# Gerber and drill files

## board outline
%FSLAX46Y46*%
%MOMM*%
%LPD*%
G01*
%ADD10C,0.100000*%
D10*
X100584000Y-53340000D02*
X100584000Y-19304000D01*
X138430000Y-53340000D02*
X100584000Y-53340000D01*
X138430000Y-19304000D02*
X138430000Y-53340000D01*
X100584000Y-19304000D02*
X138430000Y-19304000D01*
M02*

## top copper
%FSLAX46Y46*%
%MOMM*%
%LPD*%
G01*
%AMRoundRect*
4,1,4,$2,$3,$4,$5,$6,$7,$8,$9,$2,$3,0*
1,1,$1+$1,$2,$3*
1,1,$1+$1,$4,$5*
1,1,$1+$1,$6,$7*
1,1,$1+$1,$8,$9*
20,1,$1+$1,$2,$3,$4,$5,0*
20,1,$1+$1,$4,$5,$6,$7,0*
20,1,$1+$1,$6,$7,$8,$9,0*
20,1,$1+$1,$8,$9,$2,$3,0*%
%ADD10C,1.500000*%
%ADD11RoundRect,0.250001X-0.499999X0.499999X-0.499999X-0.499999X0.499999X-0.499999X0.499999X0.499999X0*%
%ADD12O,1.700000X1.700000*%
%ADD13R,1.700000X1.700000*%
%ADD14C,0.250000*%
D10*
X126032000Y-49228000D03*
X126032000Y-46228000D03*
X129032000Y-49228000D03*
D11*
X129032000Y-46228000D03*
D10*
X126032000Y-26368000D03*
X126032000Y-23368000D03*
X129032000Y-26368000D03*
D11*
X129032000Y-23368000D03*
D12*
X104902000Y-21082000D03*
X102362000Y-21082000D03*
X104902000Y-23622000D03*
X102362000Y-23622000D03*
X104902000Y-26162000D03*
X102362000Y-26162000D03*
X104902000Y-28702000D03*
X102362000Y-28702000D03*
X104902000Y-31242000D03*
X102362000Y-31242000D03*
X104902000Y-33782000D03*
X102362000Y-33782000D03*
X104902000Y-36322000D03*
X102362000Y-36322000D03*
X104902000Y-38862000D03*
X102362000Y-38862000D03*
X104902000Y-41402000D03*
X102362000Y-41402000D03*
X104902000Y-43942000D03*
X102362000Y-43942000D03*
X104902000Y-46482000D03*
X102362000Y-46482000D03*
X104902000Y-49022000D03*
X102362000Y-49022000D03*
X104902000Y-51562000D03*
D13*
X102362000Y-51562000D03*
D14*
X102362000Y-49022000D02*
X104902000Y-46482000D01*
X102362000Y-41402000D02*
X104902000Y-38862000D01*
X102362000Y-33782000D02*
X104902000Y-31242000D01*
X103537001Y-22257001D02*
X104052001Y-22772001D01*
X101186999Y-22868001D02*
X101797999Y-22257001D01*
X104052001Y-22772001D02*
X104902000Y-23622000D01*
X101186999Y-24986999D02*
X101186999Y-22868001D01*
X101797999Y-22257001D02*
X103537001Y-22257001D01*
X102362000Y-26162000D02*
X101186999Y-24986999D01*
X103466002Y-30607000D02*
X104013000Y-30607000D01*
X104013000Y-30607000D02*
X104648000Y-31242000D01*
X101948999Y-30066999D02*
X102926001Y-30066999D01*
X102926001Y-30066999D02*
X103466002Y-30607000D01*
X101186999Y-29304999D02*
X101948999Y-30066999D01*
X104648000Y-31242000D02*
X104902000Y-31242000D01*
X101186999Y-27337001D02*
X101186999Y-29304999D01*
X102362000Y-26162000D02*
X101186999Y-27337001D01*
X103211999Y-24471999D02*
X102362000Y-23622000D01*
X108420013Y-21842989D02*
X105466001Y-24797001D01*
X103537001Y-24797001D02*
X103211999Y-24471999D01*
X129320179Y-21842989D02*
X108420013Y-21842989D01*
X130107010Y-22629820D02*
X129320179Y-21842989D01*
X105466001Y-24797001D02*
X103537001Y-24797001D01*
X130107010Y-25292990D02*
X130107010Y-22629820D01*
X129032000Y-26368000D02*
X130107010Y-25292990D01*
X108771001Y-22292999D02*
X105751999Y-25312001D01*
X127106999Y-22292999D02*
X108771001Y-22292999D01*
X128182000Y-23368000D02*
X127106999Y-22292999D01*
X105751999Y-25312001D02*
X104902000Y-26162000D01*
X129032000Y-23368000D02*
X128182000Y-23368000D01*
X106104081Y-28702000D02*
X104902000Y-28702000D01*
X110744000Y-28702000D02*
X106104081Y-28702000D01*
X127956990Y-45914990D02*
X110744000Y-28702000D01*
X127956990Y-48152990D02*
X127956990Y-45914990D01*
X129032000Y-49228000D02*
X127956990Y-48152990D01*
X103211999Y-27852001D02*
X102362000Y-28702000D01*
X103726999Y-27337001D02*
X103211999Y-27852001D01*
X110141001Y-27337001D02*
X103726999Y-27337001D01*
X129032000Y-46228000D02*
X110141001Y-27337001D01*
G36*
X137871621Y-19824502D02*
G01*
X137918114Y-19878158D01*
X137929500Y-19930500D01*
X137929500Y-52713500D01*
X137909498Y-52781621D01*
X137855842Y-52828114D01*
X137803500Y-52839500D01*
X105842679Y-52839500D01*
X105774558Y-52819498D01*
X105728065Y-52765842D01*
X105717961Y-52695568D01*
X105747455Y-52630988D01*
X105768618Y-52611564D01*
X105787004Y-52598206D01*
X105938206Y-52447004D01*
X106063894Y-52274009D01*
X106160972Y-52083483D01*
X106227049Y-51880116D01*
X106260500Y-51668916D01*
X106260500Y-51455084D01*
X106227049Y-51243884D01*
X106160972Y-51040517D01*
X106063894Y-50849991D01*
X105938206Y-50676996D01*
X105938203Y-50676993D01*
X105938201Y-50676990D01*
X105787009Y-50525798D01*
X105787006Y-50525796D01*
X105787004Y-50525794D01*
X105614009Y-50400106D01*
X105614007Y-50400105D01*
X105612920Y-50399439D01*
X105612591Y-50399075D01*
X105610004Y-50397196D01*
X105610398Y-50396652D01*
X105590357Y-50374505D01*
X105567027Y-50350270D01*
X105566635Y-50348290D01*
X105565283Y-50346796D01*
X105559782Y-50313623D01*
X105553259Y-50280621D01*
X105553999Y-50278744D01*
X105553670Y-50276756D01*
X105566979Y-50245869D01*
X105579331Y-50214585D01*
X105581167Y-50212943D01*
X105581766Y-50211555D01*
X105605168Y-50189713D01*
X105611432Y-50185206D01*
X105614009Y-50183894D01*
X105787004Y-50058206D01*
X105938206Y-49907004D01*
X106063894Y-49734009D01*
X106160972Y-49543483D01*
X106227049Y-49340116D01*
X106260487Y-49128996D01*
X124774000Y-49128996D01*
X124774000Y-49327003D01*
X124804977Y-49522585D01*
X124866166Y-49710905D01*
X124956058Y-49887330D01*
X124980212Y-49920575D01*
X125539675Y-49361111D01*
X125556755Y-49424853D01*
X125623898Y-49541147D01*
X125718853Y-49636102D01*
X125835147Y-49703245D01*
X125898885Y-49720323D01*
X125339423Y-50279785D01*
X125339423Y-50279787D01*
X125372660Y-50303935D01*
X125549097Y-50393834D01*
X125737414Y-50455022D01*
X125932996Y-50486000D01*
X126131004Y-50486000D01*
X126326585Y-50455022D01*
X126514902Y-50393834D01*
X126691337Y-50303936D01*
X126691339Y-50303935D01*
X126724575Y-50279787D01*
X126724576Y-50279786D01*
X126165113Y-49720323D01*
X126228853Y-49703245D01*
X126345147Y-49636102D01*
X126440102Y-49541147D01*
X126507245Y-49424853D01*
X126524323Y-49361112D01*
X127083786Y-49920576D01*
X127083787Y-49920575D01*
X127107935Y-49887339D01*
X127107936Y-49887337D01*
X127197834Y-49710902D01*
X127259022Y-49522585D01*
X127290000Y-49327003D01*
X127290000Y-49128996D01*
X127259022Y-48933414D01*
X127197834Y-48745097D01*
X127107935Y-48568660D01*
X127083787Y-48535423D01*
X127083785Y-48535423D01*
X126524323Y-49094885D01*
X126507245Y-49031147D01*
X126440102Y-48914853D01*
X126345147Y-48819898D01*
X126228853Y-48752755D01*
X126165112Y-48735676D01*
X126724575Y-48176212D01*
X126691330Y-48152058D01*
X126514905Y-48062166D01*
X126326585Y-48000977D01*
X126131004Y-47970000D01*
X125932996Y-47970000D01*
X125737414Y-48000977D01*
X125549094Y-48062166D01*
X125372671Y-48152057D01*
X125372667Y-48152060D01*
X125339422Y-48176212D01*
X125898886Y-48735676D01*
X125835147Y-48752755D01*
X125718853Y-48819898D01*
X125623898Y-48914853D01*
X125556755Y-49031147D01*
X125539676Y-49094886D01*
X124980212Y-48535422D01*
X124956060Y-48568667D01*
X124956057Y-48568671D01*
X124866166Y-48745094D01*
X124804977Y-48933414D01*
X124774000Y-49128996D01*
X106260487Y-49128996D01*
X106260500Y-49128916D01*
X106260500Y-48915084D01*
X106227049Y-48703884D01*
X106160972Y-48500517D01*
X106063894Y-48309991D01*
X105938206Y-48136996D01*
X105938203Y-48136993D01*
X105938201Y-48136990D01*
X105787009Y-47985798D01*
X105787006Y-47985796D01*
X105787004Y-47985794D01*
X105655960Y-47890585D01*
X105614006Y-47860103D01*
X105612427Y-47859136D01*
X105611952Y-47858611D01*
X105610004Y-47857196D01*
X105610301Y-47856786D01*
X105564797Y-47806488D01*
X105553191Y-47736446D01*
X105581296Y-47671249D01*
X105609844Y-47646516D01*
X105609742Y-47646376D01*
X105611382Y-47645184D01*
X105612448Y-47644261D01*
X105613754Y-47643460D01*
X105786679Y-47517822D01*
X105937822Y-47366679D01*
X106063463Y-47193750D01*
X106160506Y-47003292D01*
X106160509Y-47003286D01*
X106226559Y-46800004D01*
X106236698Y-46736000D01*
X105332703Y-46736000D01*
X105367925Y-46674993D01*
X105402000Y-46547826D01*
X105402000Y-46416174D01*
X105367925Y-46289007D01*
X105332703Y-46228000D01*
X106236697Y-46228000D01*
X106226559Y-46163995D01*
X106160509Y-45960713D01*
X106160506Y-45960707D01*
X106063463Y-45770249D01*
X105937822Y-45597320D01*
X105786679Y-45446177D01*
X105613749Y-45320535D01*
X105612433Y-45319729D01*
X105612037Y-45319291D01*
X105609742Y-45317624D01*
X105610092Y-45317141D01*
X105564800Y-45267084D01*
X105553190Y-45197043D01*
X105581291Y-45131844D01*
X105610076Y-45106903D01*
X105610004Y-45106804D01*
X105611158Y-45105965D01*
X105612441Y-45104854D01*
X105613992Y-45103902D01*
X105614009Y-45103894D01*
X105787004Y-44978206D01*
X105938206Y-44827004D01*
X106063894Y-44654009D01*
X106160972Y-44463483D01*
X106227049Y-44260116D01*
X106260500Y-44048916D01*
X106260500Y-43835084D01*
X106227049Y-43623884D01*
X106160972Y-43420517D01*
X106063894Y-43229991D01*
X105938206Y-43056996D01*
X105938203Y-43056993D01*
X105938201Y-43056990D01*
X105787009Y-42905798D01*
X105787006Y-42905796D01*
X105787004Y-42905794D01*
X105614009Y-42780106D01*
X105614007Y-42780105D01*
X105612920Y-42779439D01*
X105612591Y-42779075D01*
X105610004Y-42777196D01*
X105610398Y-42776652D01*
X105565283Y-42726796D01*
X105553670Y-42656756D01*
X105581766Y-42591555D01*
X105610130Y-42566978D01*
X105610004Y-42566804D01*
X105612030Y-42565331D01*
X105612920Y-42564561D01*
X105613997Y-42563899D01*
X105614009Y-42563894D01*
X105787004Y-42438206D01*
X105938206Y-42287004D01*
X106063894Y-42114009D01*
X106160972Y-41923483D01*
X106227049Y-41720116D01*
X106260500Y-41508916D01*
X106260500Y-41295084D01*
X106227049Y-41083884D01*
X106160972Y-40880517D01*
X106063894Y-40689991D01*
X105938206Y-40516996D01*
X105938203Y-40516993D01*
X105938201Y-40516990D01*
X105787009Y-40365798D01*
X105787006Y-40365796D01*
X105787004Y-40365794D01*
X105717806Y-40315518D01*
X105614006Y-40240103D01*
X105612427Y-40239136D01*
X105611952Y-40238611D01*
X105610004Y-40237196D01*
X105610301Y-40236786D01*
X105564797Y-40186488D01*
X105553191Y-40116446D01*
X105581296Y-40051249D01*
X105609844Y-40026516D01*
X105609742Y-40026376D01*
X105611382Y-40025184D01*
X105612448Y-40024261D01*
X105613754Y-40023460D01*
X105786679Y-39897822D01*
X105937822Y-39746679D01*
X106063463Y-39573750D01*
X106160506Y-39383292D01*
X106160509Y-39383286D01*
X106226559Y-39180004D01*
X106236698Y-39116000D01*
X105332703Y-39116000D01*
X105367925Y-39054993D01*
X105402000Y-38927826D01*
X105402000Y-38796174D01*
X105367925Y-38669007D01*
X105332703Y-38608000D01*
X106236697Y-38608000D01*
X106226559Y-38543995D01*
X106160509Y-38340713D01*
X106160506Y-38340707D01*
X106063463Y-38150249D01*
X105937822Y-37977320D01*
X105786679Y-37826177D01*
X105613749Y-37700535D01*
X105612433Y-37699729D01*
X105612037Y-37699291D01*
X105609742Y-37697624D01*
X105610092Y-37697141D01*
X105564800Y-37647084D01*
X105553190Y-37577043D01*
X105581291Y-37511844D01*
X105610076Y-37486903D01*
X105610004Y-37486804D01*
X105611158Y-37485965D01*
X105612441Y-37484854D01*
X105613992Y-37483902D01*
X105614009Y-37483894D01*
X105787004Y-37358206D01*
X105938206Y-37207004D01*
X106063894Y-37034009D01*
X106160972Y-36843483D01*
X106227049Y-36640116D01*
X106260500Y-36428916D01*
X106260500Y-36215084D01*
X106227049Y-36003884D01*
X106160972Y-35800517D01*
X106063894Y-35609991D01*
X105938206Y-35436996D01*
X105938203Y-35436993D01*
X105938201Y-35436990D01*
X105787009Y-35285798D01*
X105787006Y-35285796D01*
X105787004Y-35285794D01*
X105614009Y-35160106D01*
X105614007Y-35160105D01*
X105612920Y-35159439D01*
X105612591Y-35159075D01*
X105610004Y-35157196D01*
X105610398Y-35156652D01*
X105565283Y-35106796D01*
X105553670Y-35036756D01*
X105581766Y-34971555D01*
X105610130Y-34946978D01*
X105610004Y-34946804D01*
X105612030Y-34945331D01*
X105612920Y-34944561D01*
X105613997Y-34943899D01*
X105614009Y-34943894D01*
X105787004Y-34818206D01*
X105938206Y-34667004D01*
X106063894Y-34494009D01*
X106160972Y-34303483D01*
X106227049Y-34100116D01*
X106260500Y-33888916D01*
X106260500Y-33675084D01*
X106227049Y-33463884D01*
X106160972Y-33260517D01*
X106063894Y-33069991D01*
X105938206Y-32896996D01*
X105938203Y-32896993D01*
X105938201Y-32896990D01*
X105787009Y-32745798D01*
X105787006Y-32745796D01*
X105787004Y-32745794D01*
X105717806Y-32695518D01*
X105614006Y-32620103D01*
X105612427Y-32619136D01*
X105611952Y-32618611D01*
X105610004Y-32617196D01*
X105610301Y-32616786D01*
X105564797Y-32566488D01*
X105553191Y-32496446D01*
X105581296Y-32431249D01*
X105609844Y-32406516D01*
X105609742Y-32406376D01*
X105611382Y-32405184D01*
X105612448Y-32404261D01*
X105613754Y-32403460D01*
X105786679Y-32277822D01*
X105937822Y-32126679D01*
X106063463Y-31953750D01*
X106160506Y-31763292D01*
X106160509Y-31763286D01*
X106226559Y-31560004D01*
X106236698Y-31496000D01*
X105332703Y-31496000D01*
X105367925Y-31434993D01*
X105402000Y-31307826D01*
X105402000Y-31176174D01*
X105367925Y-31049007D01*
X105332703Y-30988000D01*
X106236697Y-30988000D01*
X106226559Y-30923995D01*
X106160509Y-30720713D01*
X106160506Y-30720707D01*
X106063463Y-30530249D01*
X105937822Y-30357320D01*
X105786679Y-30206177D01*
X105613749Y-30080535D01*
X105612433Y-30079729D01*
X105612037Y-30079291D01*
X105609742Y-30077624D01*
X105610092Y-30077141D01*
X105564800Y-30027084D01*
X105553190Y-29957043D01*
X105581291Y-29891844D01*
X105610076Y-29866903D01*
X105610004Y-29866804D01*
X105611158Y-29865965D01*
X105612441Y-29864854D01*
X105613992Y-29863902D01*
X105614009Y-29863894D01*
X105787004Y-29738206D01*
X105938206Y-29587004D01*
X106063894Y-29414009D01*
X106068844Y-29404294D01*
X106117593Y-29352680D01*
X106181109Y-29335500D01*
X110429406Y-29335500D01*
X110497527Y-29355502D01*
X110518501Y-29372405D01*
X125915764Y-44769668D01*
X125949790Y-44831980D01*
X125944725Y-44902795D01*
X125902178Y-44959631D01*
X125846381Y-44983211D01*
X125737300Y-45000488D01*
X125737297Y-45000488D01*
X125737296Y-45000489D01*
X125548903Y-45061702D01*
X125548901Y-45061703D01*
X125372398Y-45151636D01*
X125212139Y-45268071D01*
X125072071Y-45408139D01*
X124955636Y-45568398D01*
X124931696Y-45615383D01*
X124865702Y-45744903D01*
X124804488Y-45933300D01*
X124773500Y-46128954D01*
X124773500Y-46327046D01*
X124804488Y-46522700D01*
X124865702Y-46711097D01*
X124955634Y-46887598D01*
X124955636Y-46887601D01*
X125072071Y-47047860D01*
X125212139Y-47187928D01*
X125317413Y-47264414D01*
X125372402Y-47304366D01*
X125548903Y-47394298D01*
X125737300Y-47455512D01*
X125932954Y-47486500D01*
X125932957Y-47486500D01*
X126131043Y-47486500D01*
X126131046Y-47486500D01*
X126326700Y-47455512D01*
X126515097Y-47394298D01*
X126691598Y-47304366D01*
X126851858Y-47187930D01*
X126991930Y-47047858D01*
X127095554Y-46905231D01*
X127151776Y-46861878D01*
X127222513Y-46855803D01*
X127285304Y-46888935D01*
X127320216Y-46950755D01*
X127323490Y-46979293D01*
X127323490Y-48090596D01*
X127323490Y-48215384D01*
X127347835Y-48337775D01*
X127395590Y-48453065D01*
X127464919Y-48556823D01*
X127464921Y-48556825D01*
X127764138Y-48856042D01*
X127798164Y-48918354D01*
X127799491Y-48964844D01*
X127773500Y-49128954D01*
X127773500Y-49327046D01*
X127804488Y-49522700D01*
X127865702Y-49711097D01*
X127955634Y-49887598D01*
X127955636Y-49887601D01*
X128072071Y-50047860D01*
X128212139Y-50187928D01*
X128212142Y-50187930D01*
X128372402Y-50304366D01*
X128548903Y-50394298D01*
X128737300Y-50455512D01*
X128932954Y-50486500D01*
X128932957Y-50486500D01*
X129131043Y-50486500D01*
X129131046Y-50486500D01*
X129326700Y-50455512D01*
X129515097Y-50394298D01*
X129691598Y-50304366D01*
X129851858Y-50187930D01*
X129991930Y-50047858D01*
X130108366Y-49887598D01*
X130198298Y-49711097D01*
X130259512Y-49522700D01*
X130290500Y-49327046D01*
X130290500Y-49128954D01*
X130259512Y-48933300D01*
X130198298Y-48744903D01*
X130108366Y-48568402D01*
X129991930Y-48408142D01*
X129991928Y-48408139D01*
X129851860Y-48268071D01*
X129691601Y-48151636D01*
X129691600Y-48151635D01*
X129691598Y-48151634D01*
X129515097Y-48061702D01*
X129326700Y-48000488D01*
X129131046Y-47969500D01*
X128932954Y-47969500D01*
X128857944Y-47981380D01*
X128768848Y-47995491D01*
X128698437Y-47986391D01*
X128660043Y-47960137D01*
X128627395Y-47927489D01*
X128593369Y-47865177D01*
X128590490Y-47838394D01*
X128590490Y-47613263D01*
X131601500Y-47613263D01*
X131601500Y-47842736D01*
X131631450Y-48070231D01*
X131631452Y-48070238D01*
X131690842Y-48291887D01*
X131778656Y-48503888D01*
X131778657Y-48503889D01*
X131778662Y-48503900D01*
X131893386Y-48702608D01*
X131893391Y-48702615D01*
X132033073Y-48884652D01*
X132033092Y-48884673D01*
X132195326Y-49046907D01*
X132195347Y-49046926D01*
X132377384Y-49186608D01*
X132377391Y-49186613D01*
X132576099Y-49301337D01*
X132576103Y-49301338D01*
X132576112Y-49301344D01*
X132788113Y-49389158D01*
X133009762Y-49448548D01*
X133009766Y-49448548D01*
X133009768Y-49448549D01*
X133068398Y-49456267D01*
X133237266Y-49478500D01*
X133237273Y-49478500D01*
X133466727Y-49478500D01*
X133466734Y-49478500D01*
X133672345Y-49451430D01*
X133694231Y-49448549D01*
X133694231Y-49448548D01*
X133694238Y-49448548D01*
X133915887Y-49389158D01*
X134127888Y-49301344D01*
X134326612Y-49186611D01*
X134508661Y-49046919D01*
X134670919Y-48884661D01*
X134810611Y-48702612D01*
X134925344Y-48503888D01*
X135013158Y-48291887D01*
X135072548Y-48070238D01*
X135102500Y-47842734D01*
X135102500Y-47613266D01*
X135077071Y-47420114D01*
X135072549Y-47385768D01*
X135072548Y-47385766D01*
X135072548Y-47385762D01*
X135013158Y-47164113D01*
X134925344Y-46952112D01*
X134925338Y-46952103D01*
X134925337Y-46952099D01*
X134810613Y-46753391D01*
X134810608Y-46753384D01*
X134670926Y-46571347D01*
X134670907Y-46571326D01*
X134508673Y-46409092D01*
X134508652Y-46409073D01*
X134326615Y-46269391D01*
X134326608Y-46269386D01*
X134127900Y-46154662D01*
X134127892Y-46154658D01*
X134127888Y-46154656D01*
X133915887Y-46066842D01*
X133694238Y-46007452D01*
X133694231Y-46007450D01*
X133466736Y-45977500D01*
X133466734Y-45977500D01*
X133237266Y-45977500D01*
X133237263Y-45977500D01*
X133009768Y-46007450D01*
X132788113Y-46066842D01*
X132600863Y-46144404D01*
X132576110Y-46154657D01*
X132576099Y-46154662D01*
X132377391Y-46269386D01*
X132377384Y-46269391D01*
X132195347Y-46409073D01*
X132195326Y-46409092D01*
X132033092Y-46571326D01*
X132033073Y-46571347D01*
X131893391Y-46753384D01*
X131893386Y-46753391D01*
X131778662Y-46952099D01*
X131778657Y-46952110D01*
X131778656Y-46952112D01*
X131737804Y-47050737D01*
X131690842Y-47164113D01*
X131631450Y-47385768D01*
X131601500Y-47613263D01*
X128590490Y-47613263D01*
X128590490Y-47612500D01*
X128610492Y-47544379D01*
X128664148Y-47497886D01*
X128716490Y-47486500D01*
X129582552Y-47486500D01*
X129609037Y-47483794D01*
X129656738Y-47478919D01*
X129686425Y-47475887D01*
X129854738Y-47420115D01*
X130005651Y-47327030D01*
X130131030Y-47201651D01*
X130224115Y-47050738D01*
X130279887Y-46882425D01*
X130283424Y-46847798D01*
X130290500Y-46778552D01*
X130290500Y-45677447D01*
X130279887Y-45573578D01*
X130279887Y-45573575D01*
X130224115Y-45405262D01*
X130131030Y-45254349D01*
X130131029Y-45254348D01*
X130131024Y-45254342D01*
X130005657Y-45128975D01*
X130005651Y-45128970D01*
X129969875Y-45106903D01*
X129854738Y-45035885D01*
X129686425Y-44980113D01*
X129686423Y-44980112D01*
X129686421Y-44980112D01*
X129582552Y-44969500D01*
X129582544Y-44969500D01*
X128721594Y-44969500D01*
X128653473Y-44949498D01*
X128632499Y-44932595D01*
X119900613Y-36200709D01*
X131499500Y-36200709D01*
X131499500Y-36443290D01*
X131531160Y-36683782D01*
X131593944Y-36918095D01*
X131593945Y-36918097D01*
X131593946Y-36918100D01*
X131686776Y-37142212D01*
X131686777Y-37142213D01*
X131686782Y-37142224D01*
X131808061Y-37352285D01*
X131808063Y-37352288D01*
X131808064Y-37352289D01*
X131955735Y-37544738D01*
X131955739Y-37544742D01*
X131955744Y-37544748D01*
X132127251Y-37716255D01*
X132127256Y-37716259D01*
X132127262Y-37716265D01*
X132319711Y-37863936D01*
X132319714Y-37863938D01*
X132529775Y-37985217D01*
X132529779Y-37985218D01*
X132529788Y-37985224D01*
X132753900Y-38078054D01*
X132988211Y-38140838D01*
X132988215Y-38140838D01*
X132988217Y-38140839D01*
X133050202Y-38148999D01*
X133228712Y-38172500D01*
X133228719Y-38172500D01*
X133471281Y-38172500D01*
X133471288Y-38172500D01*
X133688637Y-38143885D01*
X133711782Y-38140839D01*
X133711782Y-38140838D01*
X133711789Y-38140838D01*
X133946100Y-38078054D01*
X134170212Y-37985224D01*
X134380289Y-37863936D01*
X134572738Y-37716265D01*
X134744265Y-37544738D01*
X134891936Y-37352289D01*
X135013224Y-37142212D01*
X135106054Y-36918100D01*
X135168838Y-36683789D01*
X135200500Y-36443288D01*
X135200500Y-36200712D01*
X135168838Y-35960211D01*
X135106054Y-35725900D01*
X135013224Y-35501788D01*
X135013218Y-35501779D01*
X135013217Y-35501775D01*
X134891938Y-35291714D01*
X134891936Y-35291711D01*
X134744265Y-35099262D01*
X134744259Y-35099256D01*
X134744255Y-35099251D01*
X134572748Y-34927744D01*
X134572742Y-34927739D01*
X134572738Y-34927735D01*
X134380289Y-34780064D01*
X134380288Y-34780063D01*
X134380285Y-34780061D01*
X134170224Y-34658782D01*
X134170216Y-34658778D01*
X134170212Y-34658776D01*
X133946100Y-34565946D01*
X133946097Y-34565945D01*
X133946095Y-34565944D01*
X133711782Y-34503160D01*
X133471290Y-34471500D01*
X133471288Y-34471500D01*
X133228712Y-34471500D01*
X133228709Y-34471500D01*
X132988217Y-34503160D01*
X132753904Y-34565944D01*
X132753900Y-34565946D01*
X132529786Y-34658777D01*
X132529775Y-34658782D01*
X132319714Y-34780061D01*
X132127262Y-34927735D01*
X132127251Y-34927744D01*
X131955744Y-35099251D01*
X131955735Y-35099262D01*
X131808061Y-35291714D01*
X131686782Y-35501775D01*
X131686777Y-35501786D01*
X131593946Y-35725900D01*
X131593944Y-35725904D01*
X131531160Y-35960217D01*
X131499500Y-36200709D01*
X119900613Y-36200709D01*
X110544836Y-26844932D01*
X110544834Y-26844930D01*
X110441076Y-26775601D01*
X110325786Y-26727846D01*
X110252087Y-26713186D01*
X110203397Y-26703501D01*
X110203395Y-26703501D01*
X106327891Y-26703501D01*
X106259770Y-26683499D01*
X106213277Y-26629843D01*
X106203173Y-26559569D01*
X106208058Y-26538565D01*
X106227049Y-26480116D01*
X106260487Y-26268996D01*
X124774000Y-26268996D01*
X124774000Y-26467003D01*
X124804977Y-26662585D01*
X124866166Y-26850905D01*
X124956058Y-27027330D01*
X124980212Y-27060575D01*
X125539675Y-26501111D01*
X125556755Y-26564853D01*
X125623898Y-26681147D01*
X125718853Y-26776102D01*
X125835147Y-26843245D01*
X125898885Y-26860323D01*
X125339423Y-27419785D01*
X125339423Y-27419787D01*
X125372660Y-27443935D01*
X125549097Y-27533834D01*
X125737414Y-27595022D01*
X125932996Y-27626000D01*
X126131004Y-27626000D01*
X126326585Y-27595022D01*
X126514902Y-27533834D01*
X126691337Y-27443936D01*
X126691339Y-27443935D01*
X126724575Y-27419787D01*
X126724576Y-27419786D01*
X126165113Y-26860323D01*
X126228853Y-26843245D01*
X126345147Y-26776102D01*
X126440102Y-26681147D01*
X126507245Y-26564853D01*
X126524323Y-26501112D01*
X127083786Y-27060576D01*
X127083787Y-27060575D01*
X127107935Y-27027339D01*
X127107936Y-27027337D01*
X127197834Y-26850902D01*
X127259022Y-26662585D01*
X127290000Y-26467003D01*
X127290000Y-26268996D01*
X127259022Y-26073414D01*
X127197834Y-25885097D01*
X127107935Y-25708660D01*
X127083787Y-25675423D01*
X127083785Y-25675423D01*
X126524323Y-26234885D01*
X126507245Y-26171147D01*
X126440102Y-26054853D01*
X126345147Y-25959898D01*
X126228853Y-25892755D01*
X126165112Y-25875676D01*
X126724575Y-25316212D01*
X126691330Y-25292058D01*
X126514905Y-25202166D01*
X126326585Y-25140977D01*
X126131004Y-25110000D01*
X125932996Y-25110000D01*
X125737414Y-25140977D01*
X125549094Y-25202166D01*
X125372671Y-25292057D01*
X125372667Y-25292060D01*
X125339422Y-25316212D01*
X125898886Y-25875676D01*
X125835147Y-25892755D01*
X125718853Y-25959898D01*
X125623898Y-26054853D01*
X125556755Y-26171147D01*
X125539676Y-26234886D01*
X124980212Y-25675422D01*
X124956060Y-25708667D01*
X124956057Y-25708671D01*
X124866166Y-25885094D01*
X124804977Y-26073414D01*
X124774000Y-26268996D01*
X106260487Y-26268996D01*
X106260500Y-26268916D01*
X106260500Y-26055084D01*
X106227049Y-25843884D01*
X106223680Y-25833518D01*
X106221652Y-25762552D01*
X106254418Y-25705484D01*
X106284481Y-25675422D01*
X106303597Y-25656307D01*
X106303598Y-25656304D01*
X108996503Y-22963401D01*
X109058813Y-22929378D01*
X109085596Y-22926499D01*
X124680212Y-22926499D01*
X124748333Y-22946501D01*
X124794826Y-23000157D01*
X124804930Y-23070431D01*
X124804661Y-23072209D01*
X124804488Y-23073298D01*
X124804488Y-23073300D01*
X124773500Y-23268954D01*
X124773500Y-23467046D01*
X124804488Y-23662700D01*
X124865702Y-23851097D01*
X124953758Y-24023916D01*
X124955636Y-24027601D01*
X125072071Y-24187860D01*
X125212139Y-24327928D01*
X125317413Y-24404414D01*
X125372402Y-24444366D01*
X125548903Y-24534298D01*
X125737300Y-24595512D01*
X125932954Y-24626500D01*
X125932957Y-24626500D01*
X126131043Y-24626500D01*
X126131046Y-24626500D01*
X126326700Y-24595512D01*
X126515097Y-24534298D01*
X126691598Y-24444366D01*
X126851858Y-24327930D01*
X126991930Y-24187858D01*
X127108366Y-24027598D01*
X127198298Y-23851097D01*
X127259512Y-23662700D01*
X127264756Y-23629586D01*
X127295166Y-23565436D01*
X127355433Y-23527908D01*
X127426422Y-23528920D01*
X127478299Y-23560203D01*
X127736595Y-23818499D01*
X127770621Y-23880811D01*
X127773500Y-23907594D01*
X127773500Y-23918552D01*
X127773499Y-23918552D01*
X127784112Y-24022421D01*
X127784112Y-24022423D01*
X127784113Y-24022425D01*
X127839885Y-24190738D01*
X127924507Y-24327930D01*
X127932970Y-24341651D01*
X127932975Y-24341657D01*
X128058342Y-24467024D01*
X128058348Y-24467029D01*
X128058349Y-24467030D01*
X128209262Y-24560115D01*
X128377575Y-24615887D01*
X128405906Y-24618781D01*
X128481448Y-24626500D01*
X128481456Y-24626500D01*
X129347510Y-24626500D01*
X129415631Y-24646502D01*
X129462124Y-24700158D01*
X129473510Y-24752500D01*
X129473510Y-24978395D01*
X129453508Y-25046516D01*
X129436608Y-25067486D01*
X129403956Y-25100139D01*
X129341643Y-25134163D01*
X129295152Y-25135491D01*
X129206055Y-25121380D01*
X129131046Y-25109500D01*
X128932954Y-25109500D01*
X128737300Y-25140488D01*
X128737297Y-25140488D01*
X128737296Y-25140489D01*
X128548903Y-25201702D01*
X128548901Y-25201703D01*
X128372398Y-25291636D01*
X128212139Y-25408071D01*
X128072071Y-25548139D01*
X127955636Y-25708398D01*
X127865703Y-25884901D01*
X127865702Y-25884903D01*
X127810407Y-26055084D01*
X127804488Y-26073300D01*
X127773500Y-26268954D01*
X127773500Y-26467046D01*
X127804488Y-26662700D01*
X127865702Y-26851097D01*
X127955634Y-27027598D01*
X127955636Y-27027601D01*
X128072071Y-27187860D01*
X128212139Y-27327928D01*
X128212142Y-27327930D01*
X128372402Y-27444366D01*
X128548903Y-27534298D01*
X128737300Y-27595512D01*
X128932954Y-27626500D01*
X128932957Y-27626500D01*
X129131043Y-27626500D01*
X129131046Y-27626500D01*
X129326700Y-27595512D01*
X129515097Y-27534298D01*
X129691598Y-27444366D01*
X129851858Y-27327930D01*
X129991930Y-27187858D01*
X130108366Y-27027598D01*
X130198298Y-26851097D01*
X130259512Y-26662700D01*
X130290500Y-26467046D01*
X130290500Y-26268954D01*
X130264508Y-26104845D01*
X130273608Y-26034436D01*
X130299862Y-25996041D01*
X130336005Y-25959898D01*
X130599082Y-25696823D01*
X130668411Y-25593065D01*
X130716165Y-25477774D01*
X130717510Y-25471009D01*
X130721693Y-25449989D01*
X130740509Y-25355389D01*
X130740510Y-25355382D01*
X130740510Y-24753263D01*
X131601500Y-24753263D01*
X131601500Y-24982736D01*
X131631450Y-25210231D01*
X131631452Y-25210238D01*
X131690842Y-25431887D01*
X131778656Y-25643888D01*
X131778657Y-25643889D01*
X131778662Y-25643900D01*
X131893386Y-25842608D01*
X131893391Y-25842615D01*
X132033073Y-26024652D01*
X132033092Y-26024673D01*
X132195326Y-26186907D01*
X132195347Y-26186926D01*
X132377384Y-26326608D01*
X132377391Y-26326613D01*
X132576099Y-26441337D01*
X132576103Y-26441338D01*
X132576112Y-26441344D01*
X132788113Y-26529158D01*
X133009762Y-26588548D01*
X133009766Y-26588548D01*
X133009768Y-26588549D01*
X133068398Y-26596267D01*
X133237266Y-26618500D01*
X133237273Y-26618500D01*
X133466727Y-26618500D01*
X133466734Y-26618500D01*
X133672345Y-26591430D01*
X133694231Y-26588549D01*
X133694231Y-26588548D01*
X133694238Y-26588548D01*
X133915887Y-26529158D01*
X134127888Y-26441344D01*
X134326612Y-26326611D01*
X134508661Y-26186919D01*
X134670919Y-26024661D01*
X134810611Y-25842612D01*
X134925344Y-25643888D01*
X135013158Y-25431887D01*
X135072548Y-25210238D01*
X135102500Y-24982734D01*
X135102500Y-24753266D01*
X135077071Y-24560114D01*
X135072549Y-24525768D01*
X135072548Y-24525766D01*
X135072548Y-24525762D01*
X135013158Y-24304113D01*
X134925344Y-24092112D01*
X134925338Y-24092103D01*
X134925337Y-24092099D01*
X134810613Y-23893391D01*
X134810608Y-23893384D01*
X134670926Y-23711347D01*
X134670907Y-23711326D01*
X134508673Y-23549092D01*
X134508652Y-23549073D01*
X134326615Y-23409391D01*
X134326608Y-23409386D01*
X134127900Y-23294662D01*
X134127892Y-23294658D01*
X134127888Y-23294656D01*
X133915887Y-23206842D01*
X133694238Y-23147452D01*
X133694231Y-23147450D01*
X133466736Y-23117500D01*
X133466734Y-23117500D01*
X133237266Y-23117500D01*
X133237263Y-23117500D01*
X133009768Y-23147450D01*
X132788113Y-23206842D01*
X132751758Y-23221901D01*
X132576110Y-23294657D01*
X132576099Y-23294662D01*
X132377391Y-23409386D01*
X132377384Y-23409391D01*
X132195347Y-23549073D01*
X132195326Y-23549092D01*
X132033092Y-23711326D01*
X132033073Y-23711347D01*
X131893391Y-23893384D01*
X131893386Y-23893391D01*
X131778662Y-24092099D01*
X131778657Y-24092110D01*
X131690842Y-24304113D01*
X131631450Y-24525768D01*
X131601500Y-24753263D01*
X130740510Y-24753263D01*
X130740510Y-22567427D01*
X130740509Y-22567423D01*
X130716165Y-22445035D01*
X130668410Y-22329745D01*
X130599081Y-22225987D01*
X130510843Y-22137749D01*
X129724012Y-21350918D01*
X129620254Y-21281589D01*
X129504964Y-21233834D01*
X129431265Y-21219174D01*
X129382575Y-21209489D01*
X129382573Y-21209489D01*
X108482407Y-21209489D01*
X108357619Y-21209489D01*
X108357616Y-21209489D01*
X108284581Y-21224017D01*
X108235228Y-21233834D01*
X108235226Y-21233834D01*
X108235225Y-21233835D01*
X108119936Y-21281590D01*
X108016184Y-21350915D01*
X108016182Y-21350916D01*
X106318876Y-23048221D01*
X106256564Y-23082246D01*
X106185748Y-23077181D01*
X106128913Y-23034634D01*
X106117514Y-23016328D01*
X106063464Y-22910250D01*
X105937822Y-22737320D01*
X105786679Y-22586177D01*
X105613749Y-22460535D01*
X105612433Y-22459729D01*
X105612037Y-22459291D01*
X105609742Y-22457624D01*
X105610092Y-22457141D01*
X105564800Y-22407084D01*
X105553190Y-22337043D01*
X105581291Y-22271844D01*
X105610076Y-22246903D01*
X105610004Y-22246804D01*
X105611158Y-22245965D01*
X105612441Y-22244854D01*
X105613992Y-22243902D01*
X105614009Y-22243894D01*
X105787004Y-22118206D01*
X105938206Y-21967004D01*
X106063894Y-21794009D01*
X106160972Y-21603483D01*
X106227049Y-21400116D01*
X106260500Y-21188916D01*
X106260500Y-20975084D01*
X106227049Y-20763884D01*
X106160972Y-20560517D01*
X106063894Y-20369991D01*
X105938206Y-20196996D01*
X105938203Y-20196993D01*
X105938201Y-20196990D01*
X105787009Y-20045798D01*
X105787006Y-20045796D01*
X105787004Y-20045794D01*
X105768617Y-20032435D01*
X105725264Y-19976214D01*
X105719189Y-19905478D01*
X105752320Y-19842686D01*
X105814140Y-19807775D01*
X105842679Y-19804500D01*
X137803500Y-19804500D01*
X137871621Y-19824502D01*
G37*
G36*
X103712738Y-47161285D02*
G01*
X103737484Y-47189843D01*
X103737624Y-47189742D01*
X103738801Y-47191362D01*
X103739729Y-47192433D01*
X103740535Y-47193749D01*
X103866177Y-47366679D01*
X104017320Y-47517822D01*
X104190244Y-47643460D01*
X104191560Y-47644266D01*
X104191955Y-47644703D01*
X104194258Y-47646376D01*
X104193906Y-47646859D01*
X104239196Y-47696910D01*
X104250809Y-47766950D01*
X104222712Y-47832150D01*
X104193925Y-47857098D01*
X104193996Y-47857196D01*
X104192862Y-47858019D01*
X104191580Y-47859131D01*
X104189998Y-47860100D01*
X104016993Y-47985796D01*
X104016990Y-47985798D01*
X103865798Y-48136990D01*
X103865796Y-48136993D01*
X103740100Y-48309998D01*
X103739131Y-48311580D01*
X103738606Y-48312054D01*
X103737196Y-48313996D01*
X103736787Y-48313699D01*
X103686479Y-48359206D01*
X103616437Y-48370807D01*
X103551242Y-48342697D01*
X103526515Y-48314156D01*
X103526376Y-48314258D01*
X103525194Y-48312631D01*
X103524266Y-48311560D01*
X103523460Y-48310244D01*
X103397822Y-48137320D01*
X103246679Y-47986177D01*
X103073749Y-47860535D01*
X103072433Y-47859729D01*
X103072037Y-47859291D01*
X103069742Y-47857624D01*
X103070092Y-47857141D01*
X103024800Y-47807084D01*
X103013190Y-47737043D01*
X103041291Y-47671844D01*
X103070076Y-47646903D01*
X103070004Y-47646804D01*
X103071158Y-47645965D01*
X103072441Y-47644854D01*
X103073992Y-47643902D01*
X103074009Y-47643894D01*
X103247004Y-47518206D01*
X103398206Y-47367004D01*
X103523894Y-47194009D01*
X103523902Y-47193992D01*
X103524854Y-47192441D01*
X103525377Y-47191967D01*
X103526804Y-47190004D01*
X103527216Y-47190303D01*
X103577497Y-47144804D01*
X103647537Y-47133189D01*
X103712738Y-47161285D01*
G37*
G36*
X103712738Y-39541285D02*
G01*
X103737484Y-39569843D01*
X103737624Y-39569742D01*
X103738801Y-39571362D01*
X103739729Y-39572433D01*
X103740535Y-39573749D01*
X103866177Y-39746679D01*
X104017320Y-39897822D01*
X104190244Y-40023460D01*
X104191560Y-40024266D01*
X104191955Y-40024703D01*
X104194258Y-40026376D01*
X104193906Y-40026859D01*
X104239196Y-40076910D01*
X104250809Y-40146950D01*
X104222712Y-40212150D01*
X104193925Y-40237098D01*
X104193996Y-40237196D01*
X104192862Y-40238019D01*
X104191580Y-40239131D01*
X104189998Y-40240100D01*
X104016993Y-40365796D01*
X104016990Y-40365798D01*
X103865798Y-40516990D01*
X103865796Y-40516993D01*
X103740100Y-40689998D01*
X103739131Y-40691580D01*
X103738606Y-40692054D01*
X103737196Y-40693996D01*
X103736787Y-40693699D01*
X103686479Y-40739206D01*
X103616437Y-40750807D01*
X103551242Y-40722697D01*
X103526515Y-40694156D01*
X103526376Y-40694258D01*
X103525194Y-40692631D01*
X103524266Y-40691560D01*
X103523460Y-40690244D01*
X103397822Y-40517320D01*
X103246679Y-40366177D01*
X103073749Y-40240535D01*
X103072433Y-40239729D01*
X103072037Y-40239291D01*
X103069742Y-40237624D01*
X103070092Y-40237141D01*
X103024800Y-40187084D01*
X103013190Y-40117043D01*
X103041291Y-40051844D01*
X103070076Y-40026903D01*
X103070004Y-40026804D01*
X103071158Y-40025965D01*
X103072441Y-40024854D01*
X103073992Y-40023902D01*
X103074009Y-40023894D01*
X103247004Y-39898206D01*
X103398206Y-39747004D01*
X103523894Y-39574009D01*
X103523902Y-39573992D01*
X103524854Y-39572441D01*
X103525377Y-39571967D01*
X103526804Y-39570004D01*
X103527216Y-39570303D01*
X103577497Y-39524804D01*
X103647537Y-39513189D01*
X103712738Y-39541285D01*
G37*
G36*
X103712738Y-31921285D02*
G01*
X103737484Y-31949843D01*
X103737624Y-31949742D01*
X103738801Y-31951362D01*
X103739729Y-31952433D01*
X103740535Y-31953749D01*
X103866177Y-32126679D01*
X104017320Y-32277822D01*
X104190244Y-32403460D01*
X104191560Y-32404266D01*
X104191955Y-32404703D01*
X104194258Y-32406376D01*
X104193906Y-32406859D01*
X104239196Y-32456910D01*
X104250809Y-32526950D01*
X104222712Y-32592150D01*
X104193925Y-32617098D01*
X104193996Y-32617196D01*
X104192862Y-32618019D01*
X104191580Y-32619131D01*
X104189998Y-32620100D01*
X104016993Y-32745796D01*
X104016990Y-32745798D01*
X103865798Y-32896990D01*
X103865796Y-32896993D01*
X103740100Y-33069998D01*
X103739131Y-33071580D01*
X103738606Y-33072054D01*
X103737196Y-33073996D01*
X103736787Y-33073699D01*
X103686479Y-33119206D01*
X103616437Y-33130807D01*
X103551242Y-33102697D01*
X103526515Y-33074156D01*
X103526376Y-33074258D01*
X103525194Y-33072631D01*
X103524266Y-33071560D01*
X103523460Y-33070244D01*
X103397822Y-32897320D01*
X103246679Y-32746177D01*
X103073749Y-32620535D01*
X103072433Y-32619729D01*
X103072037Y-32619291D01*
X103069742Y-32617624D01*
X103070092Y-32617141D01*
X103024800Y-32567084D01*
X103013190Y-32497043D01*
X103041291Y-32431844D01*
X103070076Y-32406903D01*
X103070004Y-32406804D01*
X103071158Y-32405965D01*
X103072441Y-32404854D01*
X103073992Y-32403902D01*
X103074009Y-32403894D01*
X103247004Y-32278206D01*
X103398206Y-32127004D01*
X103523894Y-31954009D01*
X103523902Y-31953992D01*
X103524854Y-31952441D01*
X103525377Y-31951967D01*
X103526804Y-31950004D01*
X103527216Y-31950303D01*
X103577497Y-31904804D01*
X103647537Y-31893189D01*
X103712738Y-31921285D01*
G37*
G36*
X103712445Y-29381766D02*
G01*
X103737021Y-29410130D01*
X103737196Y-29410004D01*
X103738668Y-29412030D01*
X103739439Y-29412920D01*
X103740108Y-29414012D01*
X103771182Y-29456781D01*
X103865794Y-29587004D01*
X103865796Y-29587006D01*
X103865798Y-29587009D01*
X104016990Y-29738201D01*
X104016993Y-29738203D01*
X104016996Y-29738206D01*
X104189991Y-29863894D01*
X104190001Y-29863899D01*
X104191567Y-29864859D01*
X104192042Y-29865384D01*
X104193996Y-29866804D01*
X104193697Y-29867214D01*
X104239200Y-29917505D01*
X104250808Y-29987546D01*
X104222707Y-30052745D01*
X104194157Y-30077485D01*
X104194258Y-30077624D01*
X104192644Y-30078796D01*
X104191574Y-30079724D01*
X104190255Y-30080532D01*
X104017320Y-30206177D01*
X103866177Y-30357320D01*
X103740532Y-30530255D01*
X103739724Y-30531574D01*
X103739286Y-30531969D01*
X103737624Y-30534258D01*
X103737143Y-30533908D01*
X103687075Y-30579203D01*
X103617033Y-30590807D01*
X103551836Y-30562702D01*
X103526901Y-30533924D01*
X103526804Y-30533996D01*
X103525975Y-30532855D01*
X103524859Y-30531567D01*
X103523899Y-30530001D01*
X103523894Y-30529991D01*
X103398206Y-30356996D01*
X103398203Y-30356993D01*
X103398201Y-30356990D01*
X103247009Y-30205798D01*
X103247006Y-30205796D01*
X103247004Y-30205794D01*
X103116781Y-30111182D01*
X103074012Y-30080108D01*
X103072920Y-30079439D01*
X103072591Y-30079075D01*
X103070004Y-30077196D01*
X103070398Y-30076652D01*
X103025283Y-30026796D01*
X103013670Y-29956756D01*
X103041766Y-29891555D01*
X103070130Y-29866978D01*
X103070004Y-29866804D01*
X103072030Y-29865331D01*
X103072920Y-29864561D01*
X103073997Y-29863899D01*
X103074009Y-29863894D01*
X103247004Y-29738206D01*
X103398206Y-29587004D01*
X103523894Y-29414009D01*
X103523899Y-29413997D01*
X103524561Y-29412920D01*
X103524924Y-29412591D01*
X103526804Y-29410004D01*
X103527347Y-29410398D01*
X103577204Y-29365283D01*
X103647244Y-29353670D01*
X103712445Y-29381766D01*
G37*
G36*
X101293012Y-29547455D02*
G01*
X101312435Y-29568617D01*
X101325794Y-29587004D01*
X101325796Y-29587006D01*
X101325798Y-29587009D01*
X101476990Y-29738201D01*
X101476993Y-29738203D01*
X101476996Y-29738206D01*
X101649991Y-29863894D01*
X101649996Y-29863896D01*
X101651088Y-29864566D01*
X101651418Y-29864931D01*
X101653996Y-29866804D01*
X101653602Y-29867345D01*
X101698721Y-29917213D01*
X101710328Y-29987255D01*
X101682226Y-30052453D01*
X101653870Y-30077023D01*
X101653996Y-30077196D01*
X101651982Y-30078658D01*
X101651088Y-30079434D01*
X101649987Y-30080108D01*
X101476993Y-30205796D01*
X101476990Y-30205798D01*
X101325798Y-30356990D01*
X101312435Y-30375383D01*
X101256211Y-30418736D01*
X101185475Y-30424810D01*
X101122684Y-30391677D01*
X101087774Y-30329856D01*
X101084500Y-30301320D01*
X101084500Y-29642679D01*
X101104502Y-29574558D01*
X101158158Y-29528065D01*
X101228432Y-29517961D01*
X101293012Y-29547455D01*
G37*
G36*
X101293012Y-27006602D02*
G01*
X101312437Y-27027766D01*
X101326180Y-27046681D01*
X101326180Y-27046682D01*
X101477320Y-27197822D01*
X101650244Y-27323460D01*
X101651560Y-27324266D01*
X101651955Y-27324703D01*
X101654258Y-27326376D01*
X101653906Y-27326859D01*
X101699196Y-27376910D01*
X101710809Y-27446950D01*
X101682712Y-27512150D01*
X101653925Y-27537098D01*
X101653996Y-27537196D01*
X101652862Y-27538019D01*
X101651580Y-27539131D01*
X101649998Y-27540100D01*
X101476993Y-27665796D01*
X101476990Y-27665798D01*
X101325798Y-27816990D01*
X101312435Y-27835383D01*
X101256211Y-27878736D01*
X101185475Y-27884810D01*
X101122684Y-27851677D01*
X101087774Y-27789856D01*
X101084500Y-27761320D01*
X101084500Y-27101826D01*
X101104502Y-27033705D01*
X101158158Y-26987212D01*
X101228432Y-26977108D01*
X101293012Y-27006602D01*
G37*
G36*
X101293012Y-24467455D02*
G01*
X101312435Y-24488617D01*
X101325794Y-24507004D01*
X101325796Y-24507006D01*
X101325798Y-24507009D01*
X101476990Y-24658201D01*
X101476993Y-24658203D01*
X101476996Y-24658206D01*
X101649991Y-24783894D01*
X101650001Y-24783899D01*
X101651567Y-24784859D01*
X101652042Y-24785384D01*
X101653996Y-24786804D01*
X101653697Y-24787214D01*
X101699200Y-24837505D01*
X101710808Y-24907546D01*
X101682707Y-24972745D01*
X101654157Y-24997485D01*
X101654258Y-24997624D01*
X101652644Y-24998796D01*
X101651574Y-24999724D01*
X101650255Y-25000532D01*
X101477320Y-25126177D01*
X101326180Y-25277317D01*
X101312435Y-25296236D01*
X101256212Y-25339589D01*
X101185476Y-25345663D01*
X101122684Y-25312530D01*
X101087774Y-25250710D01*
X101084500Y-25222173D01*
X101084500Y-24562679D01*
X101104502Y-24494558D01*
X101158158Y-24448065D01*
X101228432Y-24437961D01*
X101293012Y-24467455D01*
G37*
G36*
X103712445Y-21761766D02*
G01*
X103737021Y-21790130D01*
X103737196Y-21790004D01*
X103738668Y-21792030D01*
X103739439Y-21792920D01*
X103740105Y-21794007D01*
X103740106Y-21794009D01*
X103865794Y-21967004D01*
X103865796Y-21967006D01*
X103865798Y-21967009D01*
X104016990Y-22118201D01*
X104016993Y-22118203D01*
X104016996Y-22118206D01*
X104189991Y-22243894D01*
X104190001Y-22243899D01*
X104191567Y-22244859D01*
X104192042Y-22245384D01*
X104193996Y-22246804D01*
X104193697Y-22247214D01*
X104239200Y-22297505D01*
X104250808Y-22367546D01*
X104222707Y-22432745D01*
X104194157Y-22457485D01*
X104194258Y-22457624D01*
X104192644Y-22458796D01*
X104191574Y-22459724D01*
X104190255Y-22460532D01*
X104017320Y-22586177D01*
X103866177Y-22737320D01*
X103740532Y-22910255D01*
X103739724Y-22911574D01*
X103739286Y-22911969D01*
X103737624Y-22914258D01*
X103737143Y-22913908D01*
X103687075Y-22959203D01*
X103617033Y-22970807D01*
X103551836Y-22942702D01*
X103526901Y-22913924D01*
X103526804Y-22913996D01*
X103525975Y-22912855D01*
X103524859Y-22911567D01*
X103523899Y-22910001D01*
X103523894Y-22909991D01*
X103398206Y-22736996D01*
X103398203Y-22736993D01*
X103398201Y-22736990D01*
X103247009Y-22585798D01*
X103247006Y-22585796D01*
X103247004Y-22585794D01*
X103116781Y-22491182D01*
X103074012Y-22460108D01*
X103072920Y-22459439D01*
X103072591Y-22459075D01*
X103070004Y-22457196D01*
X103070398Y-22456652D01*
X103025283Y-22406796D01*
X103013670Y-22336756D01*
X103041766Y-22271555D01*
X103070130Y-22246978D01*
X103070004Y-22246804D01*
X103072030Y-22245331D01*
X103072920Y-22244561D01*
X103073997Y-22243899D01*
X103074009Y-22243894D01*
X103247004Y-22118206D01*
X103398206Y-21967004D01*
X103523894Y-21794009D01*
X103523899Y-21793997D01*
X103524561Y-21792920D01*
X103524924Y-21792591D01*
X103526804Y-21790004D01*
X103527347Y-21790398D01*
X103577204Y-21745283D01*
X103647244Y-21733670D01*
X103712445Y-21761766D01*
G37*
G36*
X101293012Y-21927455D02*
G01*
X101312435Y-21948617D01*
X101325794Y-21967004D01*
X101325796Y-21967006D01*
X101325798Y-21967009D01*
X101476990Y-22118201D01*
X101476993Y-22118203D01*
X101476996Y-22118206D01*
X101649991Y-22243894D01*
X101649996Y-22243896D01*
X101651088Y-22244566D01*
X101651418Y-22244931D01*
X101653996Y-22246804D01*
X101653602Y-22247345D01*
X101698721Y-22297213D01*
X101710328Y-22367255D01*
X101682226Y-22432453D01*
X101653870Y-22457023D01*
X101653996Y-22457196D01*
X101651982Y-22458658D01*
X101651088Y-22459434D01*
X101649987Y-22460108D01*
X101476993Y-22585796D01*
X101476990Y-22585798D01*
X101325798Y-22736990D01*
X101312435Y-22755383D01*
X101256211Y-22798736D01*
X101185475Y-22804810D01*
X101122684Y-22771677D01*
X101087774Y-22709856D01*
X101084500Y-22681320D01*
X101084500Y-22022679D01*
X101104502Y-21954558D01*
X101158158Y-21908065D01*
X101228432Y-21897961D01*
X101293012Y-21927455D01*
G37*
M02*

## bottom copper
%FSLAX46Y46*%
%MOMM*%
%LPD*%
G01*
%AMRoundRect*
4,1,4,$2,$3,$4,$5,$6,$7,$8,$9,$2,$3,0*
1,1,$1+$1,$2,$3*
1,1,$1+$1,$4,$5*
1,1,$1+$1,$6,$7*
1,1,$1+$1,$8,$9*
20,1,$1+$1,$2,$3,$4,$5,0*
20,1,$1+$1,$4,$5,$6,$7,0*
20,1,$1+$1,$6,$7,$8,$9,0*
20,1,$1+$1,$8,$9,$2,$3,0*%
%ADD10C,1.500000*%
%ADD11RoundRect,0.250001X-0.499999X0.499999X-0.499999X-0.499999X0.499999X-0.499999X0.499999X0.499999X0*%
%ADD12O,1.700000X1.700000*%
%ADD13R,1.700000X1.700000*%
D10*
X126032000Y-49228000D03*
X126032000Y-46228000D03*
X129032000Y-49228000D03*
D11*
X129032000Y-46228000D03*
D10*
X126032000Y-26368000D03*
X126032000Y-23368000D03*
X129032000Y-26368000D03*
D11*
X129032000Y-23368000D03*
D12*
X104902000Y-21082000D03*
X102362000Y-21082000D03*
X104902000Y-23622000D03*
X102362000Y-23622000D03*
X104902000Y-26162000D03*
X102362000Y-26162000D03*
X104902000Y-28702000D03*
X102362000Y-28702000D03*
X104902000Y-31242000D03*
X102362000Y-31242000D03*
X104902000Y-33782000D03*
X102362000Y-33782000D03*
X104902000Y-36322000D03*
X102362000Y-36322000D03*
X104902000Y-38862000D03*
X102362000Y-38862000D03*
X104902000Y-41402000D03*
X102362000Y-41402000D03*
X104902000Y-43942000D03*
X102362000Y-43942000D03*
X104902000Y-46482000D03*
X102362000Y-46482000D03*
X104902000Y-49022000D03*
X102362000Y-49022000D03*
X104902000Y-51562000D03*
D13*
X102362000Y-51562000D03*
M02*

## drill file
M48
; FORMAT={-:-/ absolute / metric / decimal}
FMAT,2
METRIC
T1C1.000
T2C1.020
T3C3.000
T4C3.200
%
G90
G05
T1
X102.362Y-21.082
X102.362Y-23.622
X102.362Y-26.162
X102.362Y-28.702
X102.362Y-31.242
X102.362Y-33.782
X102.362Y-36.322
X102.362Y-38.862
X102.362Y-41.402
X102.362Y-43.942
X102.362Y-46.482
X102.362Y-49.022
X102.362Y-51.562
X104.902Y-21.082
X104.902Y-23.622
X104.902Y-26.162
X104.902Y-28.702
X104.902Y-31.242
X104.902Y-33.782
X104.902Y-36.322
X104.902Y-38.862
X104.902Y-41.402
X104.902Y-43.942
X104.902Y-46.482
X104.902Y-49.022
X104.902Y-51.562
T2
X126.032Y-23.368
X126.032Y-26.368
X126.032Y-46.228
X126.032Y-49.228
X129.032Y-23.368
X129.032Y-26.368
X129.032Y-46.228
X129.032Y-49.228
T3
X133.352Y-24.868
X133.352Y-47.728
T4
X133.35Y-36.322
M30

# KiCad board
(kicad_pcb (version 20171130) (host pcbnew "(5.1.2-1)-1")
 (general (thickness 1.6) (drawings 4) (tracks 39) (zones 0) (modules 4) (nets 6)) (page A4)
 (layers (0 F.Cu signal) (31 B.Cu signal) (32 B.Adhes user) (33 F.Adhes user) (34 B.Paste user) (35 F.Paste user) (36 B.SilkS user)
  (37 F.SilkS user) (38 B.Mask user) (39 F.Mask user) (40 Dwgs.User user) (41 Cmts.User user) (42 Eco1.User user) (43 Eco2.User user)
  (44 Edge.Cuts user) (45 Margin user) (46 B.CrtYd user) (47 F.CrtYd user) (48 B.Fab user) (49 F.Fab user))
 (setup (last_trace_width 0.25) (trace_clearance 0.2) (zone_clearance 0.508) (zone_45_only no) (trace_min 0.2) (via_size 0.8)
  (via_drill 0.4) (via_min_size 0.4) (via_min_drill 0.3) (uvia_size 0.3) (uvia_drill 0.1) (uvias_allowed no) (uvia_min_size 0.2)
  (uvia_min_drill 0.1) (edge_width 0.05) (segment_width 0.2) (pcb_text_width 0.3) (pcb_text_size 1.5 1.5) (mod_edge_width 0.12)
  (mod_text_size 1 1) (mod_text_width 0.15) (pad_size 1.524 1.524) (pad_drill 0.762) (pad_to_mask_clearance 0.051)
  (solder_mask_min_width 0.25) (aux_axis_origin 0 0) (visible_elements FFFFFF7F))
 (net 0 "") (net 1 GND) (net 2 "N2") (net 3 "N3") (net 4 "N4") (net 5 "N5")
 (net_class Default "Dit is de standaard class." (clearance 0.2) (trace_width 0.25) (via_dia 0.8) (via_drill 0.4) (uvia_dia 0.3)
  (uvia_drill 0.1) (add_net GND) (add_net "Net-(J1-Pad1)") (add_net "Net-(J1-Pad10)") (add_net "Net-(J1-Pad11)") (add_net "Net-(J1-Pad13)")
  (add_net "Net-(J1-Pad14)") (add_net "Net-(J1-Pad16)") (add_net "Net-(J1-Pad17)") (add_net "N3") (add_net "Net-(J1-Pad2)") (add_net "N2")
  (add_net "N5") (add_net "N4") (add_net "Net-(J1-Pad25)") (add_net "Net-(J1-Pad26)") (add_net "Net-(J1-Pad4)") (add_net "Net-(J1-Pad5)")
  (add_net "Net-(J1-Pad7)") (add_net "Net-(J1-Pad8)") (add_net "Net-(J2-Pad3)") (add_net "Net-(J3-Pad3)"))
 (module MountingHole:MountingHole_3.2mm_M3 (layer F.Cu) (at 133.35 36.322)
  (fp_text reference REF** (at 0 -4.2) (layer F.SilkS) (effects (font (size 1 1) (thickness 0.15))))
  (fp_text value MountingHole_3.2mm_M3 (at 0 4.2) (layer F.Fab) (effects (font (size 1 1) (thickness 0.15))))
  (pad 1 np_thru_hole circle (at 0 0) (size 3.2 3.2) (drill 3.2) (layers *.Cu *.Mask)))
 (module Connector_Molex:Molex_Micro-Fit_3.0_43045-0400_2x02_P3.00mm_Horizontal (layer F.Cu) (at 129.032 46.228 270)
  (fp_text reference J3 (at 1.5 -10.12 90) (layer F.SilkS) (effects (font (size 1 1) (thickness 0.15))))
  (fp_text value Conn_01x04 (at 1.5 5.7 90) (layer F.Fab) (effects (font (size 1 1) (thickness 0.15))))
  (pad 4 thru_hole circle (at 3 3 270) (size 1.5 1.5) (drill 1.02) (layers *.Cu *.Mask) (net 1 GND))
  (pad 3 thru_hole circle (at 0 3 270) (size 1.5 1.5) (drill 1.02) (layers *.Cu *.Mask))
  (pad 2 thru_hole circle (at 3 0 270) (size 1.5 1.5) (drill 1.02) (layers *.Cu *.Mask) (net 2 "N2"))
  (pad 1 thru_hole roundrect (at 0 0 270) (size 1.5 1.5) (drill 1.02) (layers *.Cu *.Mask) (roundrect_rratio 0.166667) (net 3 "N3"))
  (pad "" np_thru_hole circle (at 1.5 -4.32 270) (size 3 3) (drill 3) (layers *.Cu *.Mask)))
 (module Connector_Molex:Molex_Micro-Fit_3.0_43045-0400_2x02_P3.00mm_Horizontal (layer F.Cu) (at 129.032 23.368 270)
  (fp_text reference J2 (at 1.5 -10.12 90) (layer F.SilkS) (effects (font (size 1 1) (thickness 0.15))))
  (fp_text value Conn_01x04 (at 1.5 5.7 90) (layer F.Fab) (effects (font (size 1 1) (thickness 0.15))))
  (pad 4 thru_hole circle (at 3 3 270) (size 1.5 1.5) (drill 1.02) (layers *.Cu *.Mask) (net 1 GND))
  (pad 3 thru_hole circle (at 0 3 270) (size 1.5 1.5) (drill 1.02) (layers *.Cu *.Mask))
  (pad 2 thru_hole circle (at 3 0 270) (size 1.5 1.5) (drill 1.02) (layers *.Cu *.Mask) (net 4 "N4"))
  (pad 1 thru_hole roundrect (at 0 0 270) (size 1.5 1.5) (drill 1.02) (layers *.Cu *.Mask) (roundrect_rratio 0.166667) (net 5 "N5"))
  (pad "" np_thru_hole circle (at 1.5 -4.32 270) (size 3 3) (drill 3) (layers *.Cu *.Mask)))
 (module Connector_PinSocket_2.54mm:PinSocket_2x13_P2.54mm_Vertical (layer F.Cu) (at 102.362 51.562 180)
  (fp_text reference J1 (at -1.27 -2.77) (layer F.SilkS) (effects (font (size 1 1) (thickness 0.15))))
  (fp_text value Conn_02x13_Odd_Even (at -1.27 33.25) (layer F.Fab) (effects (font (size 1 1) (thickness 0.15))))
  (pad 26 thru_hole oval (at -2.54 30.48 180) (size 1.7 1.7) (drill 1) (layers *.Cu *.Mask))
  (pad 25 thru_hole oval (at 0 30.48 180) (size 1.7 1.7) (drill 1) (layers *.Cu *.Mask))
  (pad 24 thru_hole oval (at -2.54 27.94 180) (size 1.7 1.7) (drill 1) (layers *.Cu *.Mask) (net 1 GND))
  (pad 23 thru_hole oval (at 0 27.94 180) (size 1.7 1.7) (drill 1) (layers *.Cu *.Mask) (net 4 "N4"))
  (pad 22 thru_hole oval (at -2.54 25.4 180) (size 1.7 1.7) (drill 1) (layers *.Cu *.Mask) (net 5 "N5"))
  (pad 21 thru_hole oval (at 0 25.4 180) (size 1.7 1.7) (drill 1) (layers *.Cu *.Mask) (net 1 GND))
  (pad 20 thru_hole oval (at -2.54 22.86 180) (size 1.7 1.7) (drill 1) (layers *.Cu *.Mask) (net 2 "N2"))
  (pad 19 thru_hole oval (at 0 22.86 180) (size 1.7 1.7) (drill 1) (layers *.Cu *.Mask) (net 3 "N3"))
  (pad 18 thru_hole oval (at -2.54 20.32 180) (size 1.7 1.7) (drill 1) (layers *.Cu *.Mask) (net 1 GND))
  (pad 17 thru_hole oval (at 0 20.32 180) (size 1.7 1.7) (drill 1) (layers *.Cu *.Mask))
  (pad 16 thru_hole oval (at -2.54 17.78 180) (size 1.7 1.7) (drill 1) (layers *.Cu *.Mask))
  (pad 15 thru_hole oval (at 0 17.78 180) (size 1.7 1.7) (drill 1) (layers *.Cu *.Mask) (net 1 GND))
  (pad 14 thru_hole oval (at -2.54 15.24 180) (size 1.7 1.7) (drill 1) (layers *.Cu *.Mask))
  (pad 13 thru_hole oval (at 0 15.24 180) (size 1.7 1.7) (drill 1) (layers *.Cu *.Mask))
  (pad 12 thru_hole oval (at -2.54 12.7 180) (size 1.7 1.7) (drill 1) (layers *.Cu *.Mask) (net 1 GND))
  (pad 11 thru_hole oval (at 0 12.7 180) (size 1.7 1.7) (drill 1) (layers *.Cu *.Mask))
  (pad 10 thru_hole oval (at -2.54 10.16 180) (size 1.7 1.7) (drill 1) (layers *.Cu *.Mask))
  (pad 9 thru_hole oval (at 0 10.16 180) (size 1.7 1.7) (drill 1) (layers *.Cu *.Mask) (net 1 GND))
  (pad 8 thru_hole oval (at -2.54 7.62 180) (size 1.7 1.7) (drill 1) (layers *.Cu *.Mask))
  (pad 7 thru_hole oval (at 0 7.62 180) (size 1.7 1.7) (drill 1) (layers *.Cu *.Mask))
  (pad 6 thru_hole oval (at -2.54 5.08 180) (size 1.7 1.7) (drill 1) (layers *.Cu *.Mask) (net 1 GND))
  (pad 5 thru_hole oval (at 0 5.08 180) (size 1.7 1.7) (drill 1) (layers *.Cu *.Mask))
  (pad 4 thru_hole oval (at -2.54 2.54 180) (size 1.7 1.7) (drill 1) (layers *.Cu *.Mask))
  (pad 3 thru_hole oval (at 0 2.54 180) (size 1.7 1.7) (drill 1) (layers *.Cu *.Mask) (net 1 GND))
  (pad 2 thru_hole oval (at -2.54 0 180) (size 1.7 1.7) (drill 1) (layers *.Cu *.Mask))
  (pad 1 thru_hole rect (at 0 0 180) (size 1.7 1.7) (drill 1) (layers *.Cu *.Mask)))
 (gr_line (start 100.584 53.34) (end 100.584 19.304) (layer Edge.Cuts) (width 0.1))
 (gr_line (start 138.43 53.34) (end 100.584 53.34) (layer Edge.Cuts) (width 0.1))
 (gr_line (start 138.43 19.304) (end 138.43 53.34) (layer Edge.Cuts) (width 0.1))
 (gr_line (start 100.584 19.304) (end 138.43 19.304) (layer Edge.Cuts) (width 0.1))
 (segment (start 102.362 49.022) (end 104.902 46.482) (width 0.25) (layer F.Cu) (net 1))
 (segment (start 102.362 41.402) (end 104.902 38.862) (width 0.25) (layer F.Cu) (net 1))
 (segment (start 102.362 33.782) (end 104.902 31.242) (width 0.25) (layer F.Cu) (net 1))
 (segment (start 103.537001 22.257001) (end 104.052001 22.772001) (width 0.25) (layer F.Cu) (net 1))
 (segment (start 101.186999 22.868001) (end 101.797999 22.257001) (width 0.25) (layer F.Cu) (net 1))
 (segment (start 104.052001 22.772001) (end 104.902 23.622) (width 0.25) (layer F.Cu) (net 1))
 (segment (start 101.186999 24.986999) (end 101.186999 22.868001) (width 0.25) (layer F.Cu) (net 1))
 (segment (start 101.797999 22.257001) (end 103.537001 22.257001) (width 0.25) (layer F.Cu) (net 1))
 (segment (start 102.362 26.162) (end 101.186999 24.986999) (width 0.25) (layer F.Cu) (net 1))
 (segment (start 103.466002 30.607) (end 104.013 30.607) (width 0.25) (layer F.Cu) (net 1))
 (segment (start 104.013 30.607) (end 104.648 31.242) (width 0.25) (layer F.Cu) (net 1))
 (segment (start 101.948999 30.066999) (end 102.926001 30.066999) (width 0.25) (layer F.Cu) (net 1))
 (segment (start 102.926001 30.066999) (end 103.466002 30.607) (width 0.25) (layer F.Cu) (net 1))
 (segment (start 101.186999 29.304999) (end 101.948999 30.066999) (width 0.25) (layer F.Cu) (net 1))
 (segment (start 104.648 31.242) (end 104.902 31.242) (width 0.25) (layer F.Cu) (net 1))
 (segment (start 101.186999 27.337001) (end 101.186999 29.304999) (width 0.25) (layer F.Cu) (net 1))
 (segment (start 102.362 26.162) (end 101.186999 27.337001) (width 0.25) (layer F.Cu) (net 1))
 (segment (start 103.211999 24.471999) (end 102.362 23.622) (width 0.25) (layer F.Cu) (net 4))
 (segment (start 108.420013 21.842989) (end 105.466001 24.797001) (width 0.25) (layer F.Cu) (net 4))
 (segment (start 103.537001 24.797001) (end 103.211999 24.471999) (width 0.25) (layer F.Cu) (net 4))
 (segment (start 129.320179 21.842989) (end 108.420013 21.842989) (width 0.25) (layer F.Cu) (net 4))
 (segment (start 130.10701 22.62982) (end 129.320179 21.842989) (width 0.25) (layer F.Cu) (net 4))
 (segment (start 105.466001 24.797001) (end 103.537001 24.797001) (width 0.25) (layer F.Cu) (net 4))
 (segment (start 130.10701 25.29299) (end 130.10701 22.62982) (width 0.25) (layer F.Cu) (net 4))
 (segment (start 129.032 26.368) (end 130.10701 25.29299) (width 0.25) (layer F.Cu) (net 4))
 (segment (start 108.771001 22.292999) (end 105.751999 25.312001) (width 0.25) (layer F.Cu) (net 5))
 (segment (start 127.106999 22.292999) (end 108.771001 22.292999) (width 0.25) (layer F.Cu) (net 5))
 (segment (start 128.182 23.368) (end 127.106999 22.292999) (width 0.25) (layer F.Cu) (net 5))
 (segment (start 105.751999 25.312001) (end 104.902 26.162) (width 0.25) (layer F.Cu) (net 5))
 (segment (start 129.032 23.368) (end 128.182 23.368) (width 0.25) (layer F.Cu) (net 5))
 (segment (start 106.104081 28.702) (end 104.902 28.702) (width 0.25) (layer F.Cu) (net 2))
 (segment (start 110.744 28.702) (end 106.104081 28.702) (width 0.25) (layer F.Cu) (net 2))
 (segment (start 127.95699 45.91499) (end 110.744 28.702) (width 0.25) (layer F.Cu) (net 2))
 (segment (start 127.95699 48.15299) (end 127.95699 45.91499) (width 0.25) (layer F.Cu) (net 2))
 (segment (start 129.032 49.228) (end 127.95699 48.15299) (width 0.25) (layer F.Cu) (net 2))
 (segment (start 103.211999 27.852001) (end 102.362 28.702) (width 0.25) (layer F.Cu) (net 3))
 (segment (start 103.726999 27.337001) (end 103.211999 27.852001) (width 0.25) (layer F.Cu) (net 3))
 (segment (start 110.141001 27.337001) (end 103.726999 27.337001) (width 0.25) (layer F.Cu) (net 3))
 (segment (start 129.032 46.228) (end 110.141001 27.337001) (width 0.25) (layer F.Cu) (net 3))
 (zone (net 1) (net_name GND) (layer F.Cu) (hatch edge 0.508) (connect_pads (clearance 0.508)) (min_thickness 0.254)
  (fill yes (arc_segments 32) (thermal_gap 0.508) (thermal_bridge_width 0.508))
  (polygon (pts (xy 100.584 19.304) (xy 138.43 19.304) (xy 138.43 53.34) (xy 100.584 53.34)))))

